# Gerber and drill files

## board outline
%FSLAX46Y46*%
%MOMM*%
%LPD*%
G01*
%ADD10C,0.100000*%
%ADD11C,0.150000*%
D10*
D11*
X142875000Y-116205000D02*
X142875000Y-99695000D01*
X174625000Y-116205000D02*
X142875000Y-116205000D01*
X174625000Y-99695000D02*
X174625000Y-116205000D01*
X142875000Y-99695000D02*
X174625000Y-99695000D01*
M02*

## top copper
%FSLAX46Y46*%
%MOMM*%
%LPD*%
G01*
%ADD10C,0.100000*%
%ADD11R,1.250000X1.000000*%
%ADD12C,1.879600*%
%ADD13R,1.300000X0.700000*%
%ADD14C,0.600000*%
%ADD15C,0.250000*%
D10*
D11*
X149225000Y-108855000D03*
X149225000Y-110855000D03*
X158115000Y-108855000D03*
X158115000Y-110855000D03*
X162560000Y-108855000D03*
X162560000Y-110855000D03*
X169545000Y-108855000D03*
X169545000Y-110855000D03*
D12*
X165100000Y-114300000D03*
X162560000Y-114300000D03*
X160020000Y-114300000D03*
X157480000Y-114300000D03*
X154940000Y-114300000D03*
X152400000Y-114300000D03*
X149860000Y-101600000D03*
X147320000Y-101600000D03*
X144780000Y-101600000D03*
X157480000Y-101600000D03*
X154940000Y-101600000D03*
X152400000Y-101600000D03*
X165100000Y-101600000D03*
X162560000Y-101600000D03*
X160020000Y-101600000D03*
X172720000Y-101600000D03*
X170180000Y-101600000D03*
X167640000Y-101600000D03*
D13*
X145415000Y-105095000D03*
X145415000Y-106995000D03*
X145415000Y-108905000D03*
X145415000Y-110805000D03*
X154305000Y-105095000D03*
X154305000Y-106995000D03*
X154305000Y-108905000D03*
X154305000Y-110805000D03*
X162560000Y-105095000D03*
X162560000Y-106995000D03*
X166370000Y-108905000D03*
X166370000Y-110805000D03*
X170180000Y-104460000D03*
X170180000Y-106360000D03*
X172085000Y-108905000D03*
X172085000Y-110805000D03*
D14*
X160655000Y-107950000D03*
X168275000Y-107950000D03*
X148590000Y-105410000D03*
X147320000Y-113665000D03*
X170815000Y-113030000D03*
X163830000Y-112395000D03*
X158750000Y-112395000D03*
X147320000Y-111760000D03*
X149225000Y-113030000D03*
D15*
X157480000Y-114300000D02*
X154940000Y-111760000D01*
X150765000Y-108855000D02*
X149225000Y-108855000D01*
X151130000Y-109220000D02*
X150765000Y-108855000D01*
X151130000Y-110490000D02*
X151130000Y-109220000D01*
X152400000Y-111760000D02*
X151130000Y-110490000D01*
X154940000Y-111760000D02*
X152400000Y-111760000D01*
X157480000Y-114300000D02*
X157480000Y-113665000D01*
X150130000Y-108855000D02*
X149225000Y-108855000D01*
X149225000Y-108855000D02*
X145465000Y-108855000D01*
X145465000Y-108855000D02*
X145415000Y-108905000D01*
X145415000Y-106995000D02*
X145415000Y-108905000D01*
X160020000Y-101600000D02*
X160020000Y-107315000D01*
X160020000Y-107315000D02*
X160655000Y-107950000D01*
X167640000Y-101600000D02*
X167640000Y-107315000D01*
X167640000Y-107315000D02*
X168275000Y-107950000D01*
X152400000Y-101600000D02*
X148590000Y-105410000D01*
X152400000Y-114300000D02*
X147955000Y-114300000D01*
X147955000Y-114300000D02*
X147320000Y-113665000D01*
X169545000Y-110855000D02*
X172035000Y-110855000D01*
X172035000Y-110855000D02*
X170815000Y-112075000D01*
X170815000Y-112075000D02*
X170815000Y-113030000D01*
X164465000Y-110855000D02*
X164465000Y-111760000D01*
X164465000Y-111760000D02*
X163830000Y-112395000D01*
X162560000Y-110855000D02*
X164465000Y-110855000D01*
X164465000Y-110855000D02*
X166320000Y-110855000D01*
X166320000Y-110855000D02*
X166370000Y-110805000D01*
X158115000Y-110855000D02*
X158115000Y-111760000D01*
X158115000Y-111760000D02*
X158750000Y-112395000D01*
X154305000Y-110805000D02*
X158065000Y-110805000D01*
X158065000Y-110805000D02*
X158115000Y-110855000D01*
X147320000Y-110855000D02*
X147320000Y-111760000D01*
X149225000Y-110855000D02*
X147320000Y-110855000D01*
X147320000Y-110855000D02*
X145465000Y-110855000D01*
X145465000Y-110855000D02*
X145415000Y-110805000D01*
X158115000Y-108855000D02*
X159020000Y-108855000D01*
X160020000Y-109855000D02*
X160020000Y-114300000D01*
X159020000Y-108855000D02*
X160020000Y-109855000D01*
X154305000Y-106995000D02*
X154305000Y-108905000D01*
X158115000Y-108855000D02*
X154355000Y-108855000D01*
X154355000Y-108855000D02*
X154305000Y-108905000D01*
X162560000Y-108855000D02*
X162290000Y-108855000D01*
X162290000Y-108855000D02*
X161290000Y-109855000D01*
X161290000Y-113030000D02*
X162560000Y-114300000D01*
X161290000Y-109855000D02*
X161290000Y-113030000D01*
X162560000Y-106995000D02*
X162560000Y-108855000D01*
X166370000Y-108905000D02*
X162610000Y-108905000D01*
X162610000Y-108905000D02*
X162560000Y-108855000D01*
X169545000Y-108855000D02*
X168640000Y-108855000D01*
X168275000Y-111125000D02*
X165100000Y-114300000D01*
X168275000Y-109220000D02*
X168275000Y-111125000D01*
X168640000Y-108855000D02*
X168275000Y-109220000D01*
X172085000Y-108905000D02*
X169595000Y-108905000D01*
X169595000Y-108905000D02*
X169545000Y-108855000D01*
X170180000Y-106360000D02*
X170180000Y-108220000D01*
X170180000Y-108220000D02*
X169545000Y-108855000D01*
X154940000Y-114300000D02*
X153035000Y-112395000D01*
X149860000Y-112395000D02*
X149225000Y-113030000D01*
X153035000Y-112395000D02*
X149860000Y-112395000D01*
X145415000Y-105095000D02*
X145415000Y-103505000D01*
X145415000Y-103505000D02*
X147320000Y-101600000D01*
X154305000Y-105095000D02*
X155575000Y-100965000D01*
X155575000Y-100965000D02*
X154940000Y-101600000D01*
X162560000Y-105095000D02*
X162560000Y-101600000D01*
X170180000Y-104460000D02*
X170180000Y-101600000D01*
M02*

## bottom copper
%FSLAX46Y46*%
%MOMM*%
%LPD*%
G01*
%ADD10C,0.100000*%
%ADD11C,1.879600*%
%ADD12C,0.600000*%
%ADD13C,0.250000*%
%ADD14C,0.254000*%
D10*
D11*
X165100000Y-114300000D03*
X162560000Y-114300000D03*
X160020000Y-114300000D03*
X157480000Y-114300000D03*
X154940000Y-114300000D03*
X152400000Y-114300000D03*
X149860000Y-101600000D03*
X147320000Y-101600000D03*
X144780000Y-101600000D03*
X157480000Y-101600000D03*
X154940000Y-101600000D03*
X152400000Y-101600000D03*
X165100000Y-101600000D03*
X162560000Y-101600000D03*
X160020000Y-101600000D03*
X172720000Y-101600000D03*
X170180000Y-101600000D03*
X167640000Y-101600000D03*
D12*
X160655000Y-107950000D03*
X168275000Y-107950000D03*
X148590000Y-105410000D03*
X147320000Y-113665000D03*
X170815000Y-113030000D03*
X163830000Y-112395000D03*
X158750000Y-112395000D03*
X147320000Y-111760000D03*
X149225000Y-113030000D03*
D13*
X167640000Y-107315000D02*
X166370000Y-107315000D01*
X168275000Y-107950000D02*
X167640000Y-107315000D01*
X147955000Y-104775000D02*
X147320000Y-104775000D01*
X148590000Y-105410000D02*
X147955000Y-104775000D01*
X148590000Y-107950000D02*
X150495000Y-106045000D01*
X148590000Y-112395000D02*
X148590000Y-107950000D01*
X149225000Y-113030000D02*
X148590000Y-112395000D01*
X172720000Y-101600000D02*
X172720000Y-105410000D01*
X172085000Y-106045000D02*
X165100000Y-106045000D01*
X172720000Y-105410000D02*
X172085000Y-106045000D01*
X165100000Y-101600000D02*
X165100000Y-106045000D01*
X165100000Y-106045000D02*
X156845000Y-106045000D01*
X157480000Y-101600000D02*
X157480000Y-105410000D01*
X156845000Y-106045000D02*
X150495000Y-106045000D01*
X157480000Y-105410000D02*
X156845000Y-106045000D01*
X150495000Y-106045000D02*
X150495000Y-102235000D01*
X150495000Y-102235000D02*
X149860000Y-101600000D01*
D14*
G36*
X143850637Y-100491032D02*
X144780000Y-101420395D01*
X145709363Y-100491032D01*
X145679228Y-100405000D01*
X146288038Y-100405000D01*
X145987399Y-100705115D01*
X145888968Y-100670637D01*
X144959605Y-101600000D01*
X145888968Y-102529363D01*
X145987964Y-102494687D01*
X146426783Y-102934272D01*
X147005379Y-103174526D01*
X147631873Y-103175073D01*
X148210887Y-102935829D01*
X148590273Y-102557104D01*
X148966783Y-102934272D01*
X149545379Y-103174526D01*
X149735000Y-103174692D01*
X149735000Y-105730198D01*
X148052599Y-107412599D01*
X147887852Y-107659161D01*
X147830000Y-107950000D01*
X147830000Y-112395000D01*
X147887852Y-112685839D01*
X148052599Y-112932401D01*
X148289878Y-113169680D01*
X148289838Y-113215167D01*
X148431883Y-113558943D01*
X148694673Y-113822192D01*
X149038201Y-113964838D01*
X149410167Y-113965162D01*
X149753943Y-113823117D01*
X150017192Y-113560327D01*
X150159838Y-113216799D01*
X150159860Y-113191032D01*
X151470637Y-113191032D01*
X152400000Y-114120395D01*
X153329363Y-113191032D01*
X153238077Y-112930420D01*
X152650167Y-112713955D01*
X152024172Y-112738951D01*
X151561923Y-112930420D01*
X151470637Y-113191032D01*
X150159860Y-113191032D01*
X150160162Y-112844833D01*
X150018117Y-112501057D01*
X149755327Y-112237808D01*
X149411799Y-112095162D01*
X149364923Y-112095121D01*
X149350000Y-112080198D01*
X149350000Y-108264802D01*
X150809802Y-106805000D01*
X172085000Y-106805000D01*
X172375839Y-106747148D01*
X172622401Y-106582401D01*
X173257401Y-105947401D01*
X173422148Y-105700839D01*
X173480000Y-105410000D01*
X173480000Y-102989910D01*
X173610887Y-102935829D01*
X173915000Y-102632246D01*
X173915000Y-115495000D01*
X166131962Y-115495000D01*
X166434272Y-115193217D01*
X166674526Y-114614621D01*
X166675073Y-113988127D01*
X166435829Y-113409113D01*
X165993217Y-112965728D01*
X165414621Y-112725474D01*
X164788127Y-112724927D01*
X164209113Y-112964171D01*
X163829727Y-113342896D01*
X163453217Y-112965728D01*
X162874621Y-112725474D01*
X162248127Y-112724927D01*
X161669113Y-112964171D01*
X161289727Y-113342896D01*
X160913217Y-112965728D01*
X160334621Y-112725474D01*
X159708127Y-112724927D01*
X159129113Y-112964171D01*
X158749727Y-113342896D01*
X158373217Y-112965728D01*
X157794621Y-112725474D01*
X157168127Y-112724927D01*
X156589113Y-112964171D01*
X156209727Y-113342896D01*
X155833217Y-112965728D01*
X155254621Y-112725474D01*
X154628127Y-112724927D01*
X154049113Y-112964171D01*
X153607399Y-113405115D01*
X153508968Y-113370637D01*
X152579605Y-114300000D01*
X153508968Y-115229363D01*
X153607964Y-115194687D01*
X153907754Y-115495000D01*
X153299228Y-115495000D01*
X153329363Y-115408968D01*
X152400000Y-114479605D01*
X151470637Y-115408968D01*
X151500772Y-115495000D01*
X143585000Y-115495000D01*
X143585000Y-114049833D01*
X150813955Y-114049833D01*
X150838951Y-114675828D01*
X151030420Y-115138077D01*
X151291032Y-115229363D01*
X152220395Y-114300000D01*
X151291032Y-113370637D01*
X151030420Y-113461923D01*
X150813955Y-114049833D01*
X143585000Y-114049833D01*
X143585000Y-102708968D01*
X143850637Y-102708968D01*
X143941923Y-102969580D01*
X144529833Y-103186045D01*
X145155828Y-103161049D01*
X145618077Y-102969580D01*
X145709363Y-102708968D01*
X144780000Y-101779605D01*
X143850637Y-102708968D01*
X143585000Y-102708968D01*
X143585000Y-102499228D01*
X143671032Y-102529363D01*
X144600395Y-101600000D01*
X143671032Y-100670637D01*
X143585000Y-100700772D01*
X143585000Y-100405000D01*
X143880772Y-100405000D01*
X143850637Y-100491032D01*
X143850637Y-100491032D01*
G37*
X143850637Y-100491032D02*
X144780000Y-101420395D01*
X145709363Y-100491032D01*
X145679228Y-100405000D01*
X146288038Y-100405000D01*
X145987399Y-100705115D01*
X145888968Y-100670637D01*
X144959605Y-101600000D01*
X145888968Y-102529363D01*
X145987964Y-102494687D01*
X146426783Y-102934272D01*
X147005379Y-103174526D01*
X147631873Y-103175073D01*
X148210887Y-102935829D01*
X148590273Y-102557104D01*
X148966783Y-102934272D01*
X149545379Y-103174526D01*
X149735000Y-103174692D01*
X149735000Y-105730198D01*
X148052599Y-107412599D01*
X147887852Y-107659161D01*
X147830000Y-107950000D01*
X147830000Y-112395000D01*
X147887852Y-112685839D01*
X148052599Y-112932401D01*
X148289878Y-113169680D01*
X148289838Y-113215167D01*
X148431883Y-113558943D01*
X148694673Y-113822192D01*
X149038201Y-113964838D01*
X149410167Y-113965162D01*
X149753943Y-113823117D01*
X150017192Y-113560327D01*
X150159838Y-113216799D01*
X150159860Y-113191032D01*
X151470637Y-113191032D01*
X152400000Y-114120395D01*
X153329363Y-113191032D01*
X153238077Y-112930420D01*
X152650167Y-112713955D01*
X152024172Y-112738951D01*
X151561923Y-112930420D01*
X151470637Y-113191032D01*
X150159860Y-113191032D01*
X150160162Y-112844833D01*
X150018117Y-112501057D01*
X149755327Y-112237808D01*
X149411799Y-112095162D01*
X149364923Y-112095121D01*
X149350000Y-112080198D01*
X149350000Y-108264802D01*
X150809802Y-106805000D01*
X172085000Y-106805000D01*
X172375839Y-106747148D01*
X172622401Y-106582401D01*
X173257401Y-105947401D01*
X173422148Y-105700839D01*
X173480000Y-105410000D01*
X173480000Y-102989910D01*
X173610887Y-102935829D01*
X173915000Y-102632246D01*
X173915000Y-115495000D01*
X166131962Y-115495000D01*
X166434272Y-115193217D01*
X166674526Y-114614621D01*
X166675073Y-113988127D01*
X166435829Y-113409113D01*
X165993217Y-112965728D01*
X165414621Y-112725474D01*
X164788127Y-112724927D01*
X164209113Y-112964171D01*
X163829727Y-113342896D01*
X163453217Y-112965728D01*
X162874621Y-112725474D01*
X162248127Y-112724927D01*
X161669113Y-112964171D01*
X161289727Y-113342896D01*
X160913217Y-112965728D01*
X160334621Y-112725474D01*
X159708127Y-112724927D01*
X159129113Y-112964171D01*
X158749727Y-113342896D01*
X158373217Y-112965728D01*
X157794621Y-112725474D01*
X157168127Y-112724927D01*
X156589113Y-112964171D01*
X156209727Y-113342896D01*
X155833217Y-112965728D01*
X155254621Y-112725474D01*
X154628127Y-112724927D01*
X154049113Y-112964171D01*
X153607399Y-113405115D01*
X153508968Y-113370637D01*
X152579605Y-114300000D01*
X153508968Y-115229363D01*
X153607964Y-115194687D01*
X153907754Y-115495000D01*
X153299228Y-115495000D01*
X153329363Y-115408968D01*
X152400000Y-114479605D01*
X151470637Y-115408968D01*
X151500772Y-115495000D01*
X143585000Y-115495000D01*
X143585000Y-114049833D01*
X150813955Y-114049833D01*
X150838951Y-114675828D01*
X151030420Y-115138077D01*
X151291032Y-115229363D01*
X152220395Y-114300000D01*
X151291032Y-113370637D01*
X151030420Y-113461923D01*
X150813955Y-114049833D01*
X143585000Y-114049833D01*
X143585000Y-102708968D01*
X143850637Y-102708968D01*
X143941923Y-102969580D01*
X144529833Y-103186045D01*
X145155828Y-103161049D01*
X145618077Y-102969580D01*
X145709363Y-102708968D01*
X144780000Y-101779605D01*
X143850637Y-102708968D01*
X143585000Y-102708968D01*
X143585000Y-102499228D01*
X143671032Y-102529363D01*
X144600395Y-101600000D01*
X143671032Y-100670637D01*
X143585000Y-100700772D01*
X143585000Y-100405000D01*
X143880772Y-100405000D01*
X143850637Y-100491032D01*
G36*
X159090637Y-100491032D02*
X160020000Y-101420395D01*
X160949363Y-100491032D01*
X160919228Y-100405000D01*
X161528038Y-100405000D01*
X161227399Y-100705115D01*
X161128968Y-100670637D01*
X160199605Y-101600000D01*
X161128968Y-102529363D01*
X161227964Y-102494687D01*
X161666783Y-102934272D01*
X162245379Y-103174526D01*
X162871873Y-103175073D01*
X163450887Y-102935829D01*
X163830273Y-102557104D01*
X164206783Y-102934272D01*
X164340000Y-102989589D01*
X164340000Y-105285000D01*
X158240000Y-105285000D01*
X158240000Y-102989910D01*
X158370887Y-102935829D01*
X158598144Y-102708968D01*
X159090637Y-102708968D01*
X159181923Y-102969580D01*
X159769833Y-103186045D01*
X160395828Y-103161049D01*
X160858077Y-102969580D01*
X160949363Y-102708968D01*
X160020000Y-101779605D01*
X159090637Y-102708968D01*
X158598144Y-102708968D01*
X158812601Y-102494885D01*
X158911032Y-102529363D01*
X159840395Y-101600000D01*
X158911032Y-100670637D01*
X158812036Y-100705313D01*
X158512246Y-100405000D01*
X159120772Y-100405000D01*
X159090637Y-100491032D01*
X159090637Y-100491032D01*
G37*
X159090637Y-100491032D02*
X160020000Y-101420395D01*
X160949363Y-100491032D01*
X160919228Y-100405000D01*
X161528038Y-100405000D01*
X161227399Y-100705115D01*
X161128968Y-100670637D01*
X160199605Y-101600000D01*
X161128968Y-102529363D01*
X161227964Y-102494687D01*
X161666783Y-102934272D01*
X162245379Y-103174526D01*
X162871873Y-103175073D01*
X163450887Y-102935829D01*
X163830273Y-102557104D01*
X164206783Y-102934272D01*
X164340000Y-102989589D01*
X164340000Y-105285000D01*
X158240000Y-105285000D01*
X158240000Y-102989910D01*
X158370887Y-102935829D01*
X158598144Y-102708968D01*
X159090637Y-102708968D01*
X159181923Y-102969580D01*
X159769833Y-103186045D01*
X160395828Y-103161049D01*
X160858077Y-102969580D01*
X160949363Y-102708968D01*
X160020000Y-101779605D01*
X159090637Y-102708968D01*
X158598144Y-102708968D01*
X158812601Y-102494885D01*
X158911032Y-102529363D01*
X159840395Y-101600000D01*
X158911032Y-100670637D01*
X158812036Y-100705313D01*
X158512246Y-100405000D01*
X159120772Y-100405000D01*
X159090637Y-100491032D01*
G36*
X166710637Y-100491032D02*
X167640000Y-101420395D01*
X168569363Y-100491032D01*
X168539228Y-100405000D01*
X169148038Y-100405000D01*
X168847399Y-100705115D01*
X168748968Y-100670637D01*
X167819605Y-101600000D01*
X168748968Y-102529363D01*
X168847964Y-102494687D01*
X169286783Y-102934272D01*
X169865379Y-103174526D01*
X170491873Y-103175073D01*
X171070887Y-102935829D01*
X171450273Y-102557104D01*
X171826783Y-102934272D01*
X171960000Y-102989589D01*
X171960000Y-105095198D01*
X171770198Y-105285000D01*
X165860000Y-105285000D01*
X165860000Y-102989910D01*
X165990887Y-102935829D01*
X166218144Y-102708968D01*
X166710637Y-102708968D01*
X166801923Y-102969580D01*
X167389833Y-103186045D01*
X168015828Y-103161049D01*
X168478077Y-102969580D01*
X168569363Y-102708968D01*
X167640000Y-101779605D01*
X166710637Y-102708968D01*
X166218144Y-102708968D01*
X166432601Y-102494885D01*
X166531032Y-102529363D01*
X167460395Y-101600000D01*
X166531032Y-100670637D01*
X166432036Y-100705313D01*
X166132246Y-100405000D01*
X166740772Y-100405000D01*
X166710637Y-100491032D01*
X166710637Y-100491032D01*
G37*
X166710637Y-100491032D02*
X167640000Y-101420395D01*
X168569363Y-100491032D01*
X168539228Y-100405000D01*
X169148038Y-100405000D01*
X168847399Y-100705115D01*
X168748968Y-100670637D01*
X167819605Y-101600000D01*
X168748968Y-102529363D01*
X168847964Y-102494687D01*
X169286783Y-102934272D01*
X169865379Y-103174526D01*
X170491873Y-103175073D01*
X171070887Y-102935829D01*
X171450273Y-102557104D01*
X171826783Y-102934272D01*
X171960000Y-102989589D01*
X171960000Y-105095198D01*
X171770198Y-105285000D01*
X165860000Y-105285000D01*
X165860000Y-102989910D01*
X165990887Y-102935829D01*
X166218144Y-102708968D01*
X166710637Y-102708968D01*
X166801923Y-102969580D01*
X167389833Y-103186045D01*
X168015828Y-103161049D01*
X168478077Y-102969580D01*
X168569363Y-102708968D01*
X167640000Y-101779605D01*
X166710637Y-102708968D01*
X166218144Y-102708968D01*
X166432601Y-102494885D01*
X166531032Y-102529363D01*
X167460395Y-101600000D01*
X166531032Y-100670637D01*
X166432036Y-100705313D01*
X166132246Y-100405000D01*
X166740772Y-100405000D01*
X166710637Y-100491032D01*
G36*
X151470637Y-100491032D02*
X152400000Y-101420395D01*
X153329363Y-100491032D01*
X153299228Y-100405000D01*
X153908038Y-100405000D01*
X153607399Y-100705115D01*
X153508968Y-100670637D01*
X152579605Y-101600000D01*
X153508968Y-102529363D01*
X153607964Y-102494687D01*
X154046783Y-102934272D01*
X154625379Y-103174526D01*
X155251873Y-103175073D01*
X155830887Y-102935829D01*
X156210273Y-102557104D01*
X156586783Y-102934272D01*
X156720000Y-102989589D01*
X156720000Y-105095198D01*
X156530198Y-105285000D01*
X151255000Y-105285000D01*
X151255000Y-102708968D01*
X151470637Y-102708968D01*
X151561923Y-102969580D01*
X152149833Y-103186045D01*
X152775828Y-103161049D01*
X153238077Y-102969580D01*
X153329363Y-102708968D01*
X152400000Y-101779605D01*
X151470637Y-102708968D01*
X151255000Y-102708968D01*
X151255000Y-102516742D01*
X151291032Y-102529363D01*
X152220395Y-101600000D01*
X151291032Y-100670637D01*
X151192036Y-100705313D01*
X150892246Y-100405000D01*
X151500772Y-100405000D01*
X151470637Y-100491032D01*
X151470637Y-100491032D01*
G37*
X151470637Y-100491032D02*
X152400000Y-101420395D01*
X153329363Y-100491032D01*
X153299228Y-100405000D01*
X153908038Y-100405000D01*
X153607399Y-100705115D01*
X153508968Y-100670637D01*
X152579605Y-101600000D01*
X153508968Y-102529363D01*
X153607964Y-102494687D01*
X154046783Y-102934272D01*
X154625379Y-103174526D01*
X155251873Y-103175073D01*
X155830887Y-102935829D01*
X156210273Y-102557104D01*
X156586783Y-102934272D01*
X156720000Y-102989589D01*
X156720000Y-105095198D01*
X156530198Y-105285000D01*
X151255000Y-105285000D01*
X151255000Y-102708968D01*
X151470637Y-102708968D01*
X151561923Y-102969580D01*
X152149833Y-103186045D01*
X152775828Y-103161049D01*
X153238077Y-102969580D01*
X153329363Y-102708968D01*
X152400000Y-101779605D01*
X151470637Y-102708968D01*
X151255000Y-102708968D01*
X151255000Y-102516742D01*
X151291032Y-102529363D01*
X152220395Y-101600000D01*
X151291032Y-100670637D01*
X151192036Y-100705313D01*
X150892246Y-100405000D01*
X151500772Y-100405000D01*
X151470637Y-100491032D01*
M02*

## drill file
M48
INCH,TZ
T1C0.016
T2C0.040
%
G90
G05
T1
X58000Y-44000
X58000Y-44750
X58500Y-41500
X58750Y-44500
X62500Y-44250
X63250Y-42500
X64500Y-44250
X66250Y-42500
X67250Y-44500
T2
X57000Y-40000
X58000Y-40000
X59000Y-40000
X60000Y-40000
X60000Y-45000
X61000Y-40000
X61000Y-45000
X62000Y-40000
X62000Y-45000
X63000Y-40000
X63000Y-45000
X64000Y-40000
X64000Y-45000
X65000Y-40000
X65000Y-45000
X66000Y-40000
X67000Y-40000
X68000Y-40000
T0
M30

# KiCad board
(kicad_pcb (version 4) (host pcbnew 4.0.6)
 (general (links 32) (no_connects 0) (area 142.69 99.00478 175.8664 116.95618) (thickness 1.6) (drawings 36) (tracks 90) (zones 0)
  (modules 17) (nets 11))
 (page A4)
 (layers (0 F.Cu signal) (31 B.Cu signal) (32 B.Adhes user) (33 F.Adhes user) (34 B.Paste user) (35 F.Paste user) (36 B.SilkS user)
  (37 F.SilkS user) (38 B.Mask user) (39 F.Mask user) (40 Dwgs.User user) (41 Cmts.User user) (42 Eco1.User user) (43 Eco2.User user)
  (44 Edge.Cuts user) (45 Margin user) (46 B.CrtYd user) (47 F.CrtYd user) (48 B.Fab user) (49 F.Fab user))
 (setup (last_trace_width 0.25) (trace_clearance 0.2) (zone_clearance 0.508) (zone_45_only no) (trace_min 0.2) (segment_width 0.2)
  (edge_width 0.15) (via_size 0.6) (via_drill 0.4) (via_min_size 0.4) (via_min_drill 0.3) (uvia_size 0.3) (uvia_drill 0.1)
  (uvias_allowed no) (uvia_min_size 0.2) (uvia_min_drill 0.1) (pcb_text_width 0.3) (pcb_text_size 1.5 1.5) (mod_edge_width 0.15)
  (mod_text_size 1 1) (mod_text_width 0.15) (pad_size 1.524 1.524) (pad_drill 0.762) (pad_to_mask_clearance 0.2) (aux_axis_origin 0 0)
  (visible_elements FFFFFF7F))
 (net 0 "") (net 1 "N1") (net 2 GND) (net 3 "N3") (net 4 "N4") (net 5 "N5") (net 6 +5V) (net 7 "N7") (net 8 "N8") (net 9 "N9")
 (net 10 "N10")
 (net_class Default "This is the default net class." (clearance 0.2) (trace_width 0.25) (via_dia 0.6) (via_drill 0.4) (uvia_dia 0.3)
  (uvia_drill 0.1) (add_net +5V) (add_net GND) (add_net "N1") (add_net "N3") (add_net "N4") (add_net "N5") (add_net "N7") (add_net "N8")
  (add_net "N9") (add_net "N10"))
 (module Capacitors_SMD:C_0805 (layer F.Cu) (at 149.225 109.855 270)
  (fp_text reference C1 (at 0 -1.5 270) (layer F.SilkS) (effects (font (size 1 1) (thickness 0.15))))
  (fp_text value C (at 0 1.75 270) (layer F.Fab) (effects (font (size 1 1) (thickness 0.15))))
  (pad 1 smd rect (at -1 0 270) (size 1 1.25) (layers F.Cu F.Paste F.Mask) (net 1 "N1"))
  (pad 2 smd rect (at 1 0 270) (size 1 1.25) (layers F.Cu F.Paste F.Mask) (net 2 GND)))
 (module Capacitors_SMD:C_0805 (layer F.Cu) (at 158.115 109.855 270)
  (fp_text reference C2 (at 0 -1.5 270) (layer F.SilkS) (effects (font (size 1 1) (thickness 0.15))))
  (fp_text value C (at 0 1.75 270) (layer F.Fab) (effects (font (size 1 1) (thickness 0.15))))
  (pad 1 smd rect (at -1 0 270) (size 1 1.25) (layers F.Cu F.Paste F.Mask) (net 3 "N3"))
  (pad 2 smd rect (at 1 0 270) (size 1 1.25) (layers F.Cu F.Paste F.Mask) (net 2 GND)))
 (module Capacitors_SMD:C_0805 (layer F.Cu) (at 162.56 109.855 270)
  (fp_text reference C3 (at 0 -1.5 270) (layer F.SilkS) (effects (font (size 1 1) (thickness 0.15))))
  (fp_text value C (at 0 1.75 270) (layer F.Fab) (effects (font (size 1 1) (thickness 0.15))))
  (pad 1 smd rect (at -1 0 270) (size 1 1.25) (layers F.Cu F.Paste F.Mask) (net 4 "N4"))
  (pad 2 smd rect (at 1 0 270) (size 1 1.25) (layers F.Cu F.Paste F.Mask) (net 2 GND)))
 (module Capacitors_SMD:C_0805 (layer F.Cu) (at 169.545 109.855 270)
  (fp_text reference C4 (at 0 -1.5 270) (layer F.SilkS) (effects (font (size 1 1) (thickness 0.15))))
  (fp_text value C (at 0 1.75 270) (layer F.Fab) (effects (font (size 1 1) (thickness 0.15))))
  (pad 1 smd rect (at -1 0 270) (size 1 1.25) (layers F.Cu F.Paste F.Mask) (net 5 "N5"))
  (pad 2 smd rect (at 1 0 270) (size 1 1.25) (layers F.Cu F.Paste F.Mask) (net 2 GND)))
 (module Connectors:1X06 (layer F.Cu) (at 165.1 114.3 180)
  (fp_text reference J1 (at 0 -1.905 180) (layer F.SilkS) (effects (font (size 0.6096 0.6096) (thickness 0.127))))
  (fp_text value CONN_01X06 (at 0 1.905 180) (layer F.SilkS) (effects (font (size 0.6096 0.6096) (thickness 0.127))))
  (pad 1 thru_hole circle (at 0 0 180) (size 1.8796 1.8796) (drill 1.016) (layers *.Cu *.Mask) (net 5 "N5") (solder_mask_margin 0.1016))
  (pad 2 thru_hole circle (at 2.54 0 180) (size 1.8796 1.8796) (drill 1.016) (layers *.Cu *.Mask) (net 4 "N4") (solder_mask_margin 0.1016))
  (pad 3 thru_hole circle (at 5.08 0 180) (size 1.8796 1.8796) (drill 1.016) (layers *.Cu *.Mask) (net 3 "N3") (solder_mask_margin 0.1016))
  (pad 4 thru_hole circle (at 7.62 0 180) (size 1.8796 1.8796) (drill 1.016) (layers *.Cu *.Mask) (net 1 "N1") (solder_mask_margin 0.1016))
  (pad 5 thru_hole circle (at 10.16 0 180) (size 1.8796 1.8796) (drill 1.016) (layers *.Cu *.Mask) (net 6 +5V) (solder_mask_margin 0.1016))
  (pad 6 thru_hole circle (at 12.7 0 180) (size 1.8796 1.8796) (drill 1.016) (layers *.Cu *.Mask) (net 2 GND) (solder_mask_margin 0.1016)))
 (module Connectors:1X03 (layer F.Cu) (at 149.86 101.6 180)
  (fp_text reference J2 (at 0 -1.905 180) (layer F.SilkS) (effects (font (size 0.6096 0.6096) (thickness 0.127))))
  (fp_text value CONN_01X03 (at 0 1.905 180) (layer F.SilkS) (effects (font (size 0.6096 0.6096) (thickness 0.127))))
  (pad 1 thru_hole circle (at 0 0 180) (size 1.8796 1.8796) (drill 1.016) (layers *.Cu *.Mask) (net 6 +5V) (solder_mask_margin 0.1016))
  (pad 2 thru_hole circle (at 2.54 0 180) (size 1.8796 1.8796) (drill 1.016) (layers *.Cu *.Mask) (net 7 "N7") (solder_mask_margin 0.1016))
  (pad 3 thru_hole circle (at 5.08 0 180) (size 1.8796 1.8796) (drill 1.016) (layers *.Cu *.Mask) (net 2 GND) (solder_mask_margin 0.1016)))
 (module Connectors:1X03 (layer F.Cu) (at 157.48 101.6 180)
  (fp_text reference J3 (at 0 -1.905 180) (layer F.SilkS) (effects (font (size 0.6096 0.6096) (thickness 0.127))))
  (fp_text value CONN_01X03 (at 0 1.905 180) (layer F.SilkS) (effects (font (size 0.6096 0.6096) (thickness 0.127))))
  (pad 1 thru_hole circle (at 0 0 180) (size 1.8796 1.8796) (drill 1.016) (layers *.Cu *.Mask) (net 6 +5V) (solder_mask_margin 0.1016))
  (pad 2 thru_hole circle (at 2.54 0 180) (size 1.8796 1.8796) (drill 1.016) (layers *.Cu *.Mask) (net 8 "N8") (solder_mask_margin 0.1016))
  (pad 3 thru_hole circle (at 5.08 0 180) (size 1.8796 1.8796) (drill 1.016) (layers *.Cu *.Mask) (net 2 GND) (solder_mask_margin 0.1016)))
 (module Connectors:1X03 (layer F.Cu) (at 165.1 101.6 180)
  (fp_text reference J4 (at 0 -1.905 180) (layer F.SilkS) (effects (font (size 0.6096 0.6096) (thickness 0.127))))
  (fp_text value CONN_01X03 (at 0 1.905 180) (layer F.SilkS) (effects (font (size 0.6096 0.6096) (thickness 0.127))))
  (pad 1 thru_hole circle (at 0 0 180) (size 1.8796 1.8796) (drill 1.016) (layers *.Cu *.Mask) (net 6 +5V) (solder_mask_margin 0.1016))
  (pad 2 thru_hole circle (at 2.54 0 180) (size 1.8796 1.8796) (drill 1.016) (layers *.Cu *.Mask) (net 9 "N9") (solder_mask_margin 0.1016))
  (pad 3 thru_hole circle (at 5.08 0 180) (size 1.8796 1.8796) (drill 1.016) (layers *.Cu *.Mask) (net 2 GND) (solder_mask_margin 0.1016)))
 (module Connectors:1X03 (layer F.Cu) (at 172.72 101.6 180)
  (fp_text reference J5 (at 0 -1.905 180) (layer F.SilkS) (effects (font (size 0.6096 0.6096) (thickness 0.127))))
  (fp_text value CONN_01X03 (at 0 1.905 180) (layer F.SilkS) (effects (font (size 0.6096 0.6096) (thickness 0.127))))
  (pad 1 thru_hole circle (at 0 0 180) (size 1.8796 1.8796) (drill 1.016) (layers *.Cu *.Mask) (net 6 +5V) (solder_mask_margin 0.1016))
  (pad 2 thru_hole circle (at 2.54 0 180) (size 1.8796 1.8796) (drill 1.016) (layers *.Cu *.Mask) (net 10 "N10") (solder_mask_margin 0.1016))
  (pad 3 thru_hole circle (at 5.08 0 180) (size 1.8796 1.8796) (drill 1.016) (layers *.Cu *.Mask) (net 2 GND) (solder_mask_margin 0.1016)))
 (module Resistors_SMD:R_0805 (layer F.Cu) (at 145.415 106.045 270)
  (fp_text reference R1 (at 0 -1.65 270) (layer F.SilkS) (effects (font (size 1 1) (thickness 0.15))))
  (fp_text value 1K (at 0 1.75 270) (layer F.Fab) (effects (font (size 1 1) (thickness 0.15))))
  (pad 1 smd rect (at -0.95 0 270) (size 0.7 1.3) (layers F.Cu F.Paste F.Mask) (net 7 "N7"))
  (pad 2 smd rect (at 0.95 0 270) (size 0.7 1.3) (layers F.Cu F.Paste F.Mask) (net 1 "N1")))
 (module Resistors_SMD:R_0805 (layer F.Cu) (at 145.415 109.855 270)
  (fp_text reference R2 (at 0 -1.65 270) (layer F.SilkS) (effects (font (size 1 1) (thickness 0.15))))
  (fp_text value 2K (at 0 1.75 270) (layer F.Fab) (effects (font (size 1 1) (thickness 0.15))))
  (pad 1 smd rect (at -0.95 0 270) (size 0.7 1.3) (layers F.Cu F.Paste F.Mask) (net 1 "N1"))
  (pad 2 smd rect (at 0.95 0 270) (size 0.7 1.3) (layers F.Cu F.Paste F.Mask) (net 2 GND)))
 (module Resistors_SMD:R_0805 (layer F.Cu) (at 154.305 106.045 270)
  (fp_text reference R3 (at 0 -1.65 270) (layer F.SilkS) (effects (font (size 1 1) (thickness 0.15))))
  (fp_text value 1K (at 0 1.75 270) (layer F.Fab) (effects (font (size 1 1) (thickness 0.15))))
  (pad 1 smd rect (at -0.95 0 270) (size 0.7 1.3) (layers F.Cu F.Paste F.Mask) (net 8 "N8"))
  (pad 2 smd rect (at 0.95 0 270) (size 0.7 1.3) (layers F.Cu F.Paste F.Mask) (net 3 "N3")))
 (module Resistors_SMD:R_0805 (layer F.Cu) (at 154.305 109.855 270)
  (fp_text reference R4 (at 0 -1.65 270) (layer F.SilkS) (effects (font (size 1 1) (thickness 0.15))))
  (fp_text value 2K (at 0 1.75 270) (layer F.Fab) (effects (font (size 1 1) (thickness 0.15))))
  (pad 1 smd rect (at -0.95 0 270) (size 0.7 1.3) (layers F.Cu F.Paste F.Mask) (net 3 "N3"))
  (pad 2 smd rect (at 0.95 0 270) (size 0.7 1.3) (layers F.Cu F.Paste F.Mask) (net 2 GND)))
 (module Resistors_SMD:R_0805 (layer F.Cu) (at 162.56 106.045 270)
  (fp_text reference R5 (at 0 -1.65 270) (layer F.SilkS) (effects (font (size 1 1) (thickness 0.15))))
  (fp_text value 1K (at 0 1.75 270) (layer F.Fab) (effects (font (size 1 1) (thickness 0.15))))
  (pad 1 smd rect (at -0.95 0 270) (size 0.7 1.3) (layers F.Cu F.Paste F.Mask) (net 9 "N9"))
  (pad 2 smd rect (at 0.95 0 270) (size 0.7 1.3) (layers F.Cu F.Paste F.Mask) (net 4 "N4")))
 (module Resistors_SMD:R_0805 (layer F.Cu) (at 166.37 109.855 270)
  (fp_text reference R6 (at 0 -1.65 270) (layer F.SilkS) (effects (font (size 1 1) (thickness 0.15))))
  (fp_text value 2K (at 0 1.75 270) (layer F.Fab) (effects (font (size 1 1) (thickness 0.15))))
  (pad 1 smd rect (at -0.95 0 270) (size 0.7 1.3) (layers F.Cu F.Paste F.Mask) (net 4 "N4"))
  (pad 2 smd rect (at 0.95 0 270) (size 0.7 1.3) (layers F.Cu F.Paste F.Mask) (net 2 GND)))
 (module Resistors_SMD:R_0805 (layer F.Cu) (at 170.18 105.41 270)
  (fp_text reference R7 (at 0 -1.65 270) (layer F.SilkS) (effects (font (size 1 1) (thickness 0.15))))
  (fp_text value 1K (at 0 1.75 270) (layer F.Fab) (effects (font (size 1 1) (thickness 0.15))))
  (pad 1 smd rect (at -0.95 0 270) (size 0.7 1.3) (layers F.Cu F.Paste F.Mask) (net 10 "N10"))
  (pad 2 smd rect (at 0.95 0 270) (size 0.7 1.3) (layers F.Cu F.Paste F.Mask) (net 5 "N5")))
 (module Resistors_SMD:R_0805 (layer F.Cu) (at 172.085 109.855 270)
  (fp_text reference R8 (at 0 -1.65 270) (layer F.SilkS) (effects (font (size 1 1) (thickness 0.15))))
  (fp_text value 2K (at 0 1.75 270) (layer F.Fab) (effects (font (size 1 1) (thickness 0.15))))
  (pad 1 smd rect (at -0.95 0 270) (size 0.7 1.3) (layers F.Cu F.Paste F.Mask) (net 5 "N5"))
  (pad 2 smd rect (at 0.95 0 270) (size 0.7 1.3) (layers F.Cu F.Paste F.Mask) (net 2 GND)))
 (gr_line (start 142.875 116.205) (end 142.875 99.695) (angle 90) (layer Edge.Cuts) (width 0.15))
 (gr_line (start 174.625 116.205) (end 142.875 116.205) (angle 90) (layer Edge.Cuts) (width 0.15))
 (gr_line (start 174.625 99.695) (end 174.625 116.205) (angle 90) (layer Edge.Cuts) (width 0.15))
 (gr_line (start 142.875 99.695) (end 174.625 99.695) (angle 90) (layer Edge.Cuts) (width 0.15))
 (segment (start 157.48 114.3) (end 154.94 111.76) (width 0.25) (layer F.Cu) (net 1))
 (segment (start 150.765 108.855) (end 149.225 108.855) (width 0.25) (layer F.Cu) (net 1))
 (segment (start 151.13 109.22) (end 150.765 108.855) (width 0.25) (layer F.Cu) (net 1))
 (segment (start 151.13 110.49) (end 151.13 109.22) (width 0.25) (layer F.Cu) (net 1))
 (segment (start 152.4 111.76) (end 151.13 110.49) (width 0.25) (layer F.Cu) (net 1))
 (segment (start 154.94 111.76) (end 152.4 111.76) (width 0.25) (layer F.Cu) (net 1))
 (segment (start 157.48 114.3) (end 157.48 113.665) (width 0.25) (layer F.Cu) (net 1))
 (segment (start 150.13 108.855) (end 149.225 108.855) (width 0.25) (layer F.Cu) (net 1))
 (segment (start 149.225 108.855) (end 145.465 108.855) (width 0.25) (layer F.Cu) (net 1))
 (segment (start 145.465 108.855) (end 145.415 108.905) (width 0.25) (layer F.Cu) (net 1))
 (segment (start 145.415 106.995) (end 145.415 108.905) (width 0.25) (layer F.Cu) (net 1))
 (segment (start 160.02 101.6) (end 160.02 107.315) (width 0.25) (layer F.Cu) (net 2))
 (via (at 160.655 107.95) (size 0.6) (drill 0.4) (layers F.Cu B.Cu) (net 2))
 (segment (start 160.02 107.315) (end 160.655 107.95) (width 0.25) (layer F.Cu) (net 2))
 (segment (start 167.64 101.6) (end 167.64 107.315) (width 0.25) (layer F.Cu) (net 2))
 (segment (start 167.64 107.315) (end 166.37 107.315) (width 0.25) (layer B.Cu) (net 2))
 (segment (start 168.275 107.95) (end 167.64 107.315) (width 0.25) (layer B.Cu) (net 2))
 (via (at 168.275 107.95) (size 0.6) (drill 0.4) (layers F.Cu B.Cu) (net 2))
 (segment (start 167.64 107.315) (end 168.275 107.95) (width 0.25) (layer F.Cu) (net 2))
 (segment (start 152.4 101.6) (end 148.59 105.41) (width 0.25) (layer F.Cu) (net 2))
 (segment (start 147.955 104.775) (end 147.32 104.775) (width 0.25) (layer B.Cu) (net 2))
 (segment (start 148.59 105.41) (end 147.955 104.775) (width 0.25) (layer B.Cu) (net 2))
 (via (at 148.59 105.41) (size 0.6) (drill 0.4) (layers F.Cu B.Cu) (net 2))
 (segment (start 152.4 114.3) (end 147.955 114.3) (width 0.25) (layer F.Cu) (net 2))
 (via (at 147.32 113.665) (size 0.6) (drill 0.4) (layers F.Cu B.Cu) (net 2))
 (segment (start 147.955 114.3) (end 147.32 113.665) (width 0.25) (layer F.Cu) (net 2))
 (segment (start 169.545 110.855) (end 172.035 110.855) (width 0.25) (layer F.Cu) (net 2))
 (segment (start 172.035 110.855) (end 170.815 112.075) (width 0.25) (layer F.Cu) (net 2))
 (segment (start 170.815 112.075) (end 170.815 113.03) (width 0.25) (layer F.Cu) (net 2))
 (via (at 170.815 113.03) (size 0.6) (drill 0.4) (layers F.Cu B.Cu) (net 2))
 (segment (start 164.465 110.855) (end 164.465 111.76) (width 0.25) (layer F.Cu) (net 2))
 (via (at 163.83 112.395) (size 0.6) (drill 0.4) (layers F.Cu B.Cu) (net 2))
 (segment (start 164.465 111.76) (end 163.83 112.395) (width 0.25) (layer F.Cu) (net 2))
 (segment (start 162.56 110.855) (end 164.465 110.855) (width 0.25) (layer F.Cu) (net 2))
 (segment (start 164.465 110.855) (end 166.32 110.855) (width 0.25) (layer F.Cu) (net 2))
 (segment (start 166.32 110.855) (end 166.37 110.805) (width 0.25) (layer F.Cu) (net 2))
 (segment (start 158.115 110.855) (end 158.115 111.76) (width 0.25) (layer F.Cu) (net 2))
 (via (at 158.75 112.395) (size 0.6) (drill 0.4) (layers F.Cu B.Cu) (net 2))
 (segment (start 158.115 111.76) (end 158.75 112.395) (width 0.25) (layer F.Cu) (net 2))
 (segment (start 154.305 110.805) (end 158.065 110.805) (width 0.25) (layer F.Cu) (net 2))
 (segment (start 158.065 110.805) (end 158.115 110.855) (width 0.25) (layer F.Cu) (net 2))
 (segment (start 147.32 110.855) (end 147.32 111.76) (width 0.25) (layer F.Cu) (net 2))
 (via (at 147.32 111.76) (size 0.6) (drill 0.4) (layers F.Cu B.Cu) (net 2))
 (segment (start 149.225 110.855) (end 147.32 110.855) (width 0.25) (layer F.Cu) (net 2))
 (segment (start 147.32 110.855) (end 145.465 110.855) (width 0.25) (layer F.Cu) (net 2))
 (segment (start 145.465 110.855) (end 145.415 110.805) (width 0.25) (layer F.Cu) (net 2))
 (segment (start 158.115 108.855) (end 159.02 108.855) (width 0.25) (layer F.Cu) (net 3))
 (segment (start 160.02 109.855) (end 160.02 114.3) (width 0.25) (layer F.Cu) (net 3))
 (segment (start 159.02 108.855) (end 160.02 109.855) (width 0.25) (layer F.Cu) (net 3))
 (segment (start 154.305 106.995) (end 154.305 108.905) (width 0.25) (layer F.Cu) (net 3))
 (segment (start 158.115 108.855) (end 154.355 108.855) (width 0.25) (layer F.Cu) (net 3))
 (segment (start 154.355 108.855) (end 154.305 108.905) (width 0.25) (layer F.Cu) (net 3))
 (segment (start 162.56 108.855) (end 162.29 108.855) (width 0.25) (layer F.Cu) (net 4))
 (segment (start 162.29 108.855) (end 161.29 109.855) (width 0.25) (layer F.Cu) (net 4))
 (segment (start 161.29 113.03) (end 162.56 114.3) (width 0.25) (layer F.Cu) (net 4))
 (segment (start 161.29 109.855) (end 161.29 113.03) (width 0.25) (layer F.Cu) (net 4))
 (segment (start 162.56 106.995) (end 162.56 108.855) (width 0.25) (layer F.Cu) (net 4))
 (segment (start 166.37 108.905) (end 162.61 108.905) (width 0.25) (layer F.Cu) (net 4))
 (segment (start 162.61 108.905) (end 162.56 108.855) (width 0.25) (layer F.Cu) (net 4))
 (segment (start 169.545 108.855) (end 168.64 108.855) (width 0.25) (layer F.Cu) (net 5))
 (segment (start 168.275 111.125) (end 165.1 114.3) (width 0.25) (layer F.Cu) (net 5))
 (segment (start 168.275 109.22) (end 168.275 111.125) (width 0.25) (layer F.Cu) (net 5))
 (segment (start 168.64 108.855) (end 168.275 109.22) (width 0.25) (layer F.Cu) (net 5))
 (segment (start 172.085 108.905) (end 169.595 108.905) (width 0.25) (layer F.Cu) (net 5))
 (segment (start 169.595 108.905) (end 169.545 108.855) (width 0.25) (layer F.Cu) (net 5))
 (segment (start 170.18 106.36) (end 170.18 108.22) (width 0.25) (layer F.Cu) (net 5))
 (segment (start 170.18 108.22) (end 169.545 108.855) (width 0.25) (layer F.Cu) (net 5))
 (segment (start 154.94 114.3) (end 153.035 112.395) (width 0.25) (layer F.Cu) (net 6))
 (segment (start 148.59 107.95) (end 150.495 106.045) (width 0.25) (layer B.Cu) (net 6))
 (segment (start 148.59 112.395) (end 148.59 107.95) (width 0.25) (layer B.Cu) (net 6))
 (segment (start 149.225 113.03) (end 148.59 112.395) (width 0.25) (layer B.Cu) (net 6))
 (via (at 149.225 113.03) (size 0.6) (drill 0.4) (layers F.Cu B.Cu) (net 6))
 (segment (start 149.86 112.395) (end 149.225 113.03) (width 0.25) (layer F.Cu) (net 6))
 (segment (start 153.035 112.395) (end 149.86 112.395) (width 0.25) (layer F.Cu) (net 6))
 (segment (start 172.72 101.6) (end 172.72 105.41) (width 0.25) (layer B.Cu) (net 6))
 (segment (start 172.085 106.045) (end 165.1 106.045) (width 0.25) (layer B.Cu) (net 6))
 (segment (start 172.72 105.41) (end 172.085 106.045) (width 0.25) (layer B.Cu) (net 6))
 (segment (start 165.1 101.6) (end 165.1 106.045) (width 0.25) (layer B.Cu) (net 6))
 (segment (start 165.1 106.045) (end 156.845 106.045) (width 0.25) (layer B.Cu) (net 6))
 (segment (start 157.48 101.6) (end 157.48 105.41) (width 0.25) (layer B.Cu) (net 6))
 (segment (start 156.845 106.045) (end 150.495 106.045) (width 0.25) (layer B.Cu) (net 6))
 (segment (start 157.48 105.41) (end 156.845 106.045) (width 0.25) (layer B.Cu) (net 6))
 (segment (start 150.495 106.045) (end 150.495 102.235) (width 0.25) (layer B.Cu) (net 6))
 (segment (start 150.495 102.235) (end 149.86 101.6) (width 0.25) (layer B.Cu) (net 6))
 (segment (start 145.415 105.095) (end 145.415 103.505) (width 0.25) (layer F.Cu) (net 7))
 (segment (start 145.415 103.505) (end 147.32 101.6) (width 0.25) (layer F.Cu) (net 7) (status 20))
 (segment (start 154.305 105.095) (end 155.575 100.965) (width 0.25) (layer F.Cu) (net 8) (status 20))
 (segment (start 155.575 100.965) (end 154.94 101.6) (width 0.25) (layer F.Cu) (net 8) (status 30))
 (segment (start 162.56 105.095) (end 162.56 101.6) (width 0.25) (layer F.Cu) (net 9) (status 20))
 (segment (start 170.18 104.46) (end 170.18 101.6) (width 0.25) (layer F.Cu) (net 10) (status 20))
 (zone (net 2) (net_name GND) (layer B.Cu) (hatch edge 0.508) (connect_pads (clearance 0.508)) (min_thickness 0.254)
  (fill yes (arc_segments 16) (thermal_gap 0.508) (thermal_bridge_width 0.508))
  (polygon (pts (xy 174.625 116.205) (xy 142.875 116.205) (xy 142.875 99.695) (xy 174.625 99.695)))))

